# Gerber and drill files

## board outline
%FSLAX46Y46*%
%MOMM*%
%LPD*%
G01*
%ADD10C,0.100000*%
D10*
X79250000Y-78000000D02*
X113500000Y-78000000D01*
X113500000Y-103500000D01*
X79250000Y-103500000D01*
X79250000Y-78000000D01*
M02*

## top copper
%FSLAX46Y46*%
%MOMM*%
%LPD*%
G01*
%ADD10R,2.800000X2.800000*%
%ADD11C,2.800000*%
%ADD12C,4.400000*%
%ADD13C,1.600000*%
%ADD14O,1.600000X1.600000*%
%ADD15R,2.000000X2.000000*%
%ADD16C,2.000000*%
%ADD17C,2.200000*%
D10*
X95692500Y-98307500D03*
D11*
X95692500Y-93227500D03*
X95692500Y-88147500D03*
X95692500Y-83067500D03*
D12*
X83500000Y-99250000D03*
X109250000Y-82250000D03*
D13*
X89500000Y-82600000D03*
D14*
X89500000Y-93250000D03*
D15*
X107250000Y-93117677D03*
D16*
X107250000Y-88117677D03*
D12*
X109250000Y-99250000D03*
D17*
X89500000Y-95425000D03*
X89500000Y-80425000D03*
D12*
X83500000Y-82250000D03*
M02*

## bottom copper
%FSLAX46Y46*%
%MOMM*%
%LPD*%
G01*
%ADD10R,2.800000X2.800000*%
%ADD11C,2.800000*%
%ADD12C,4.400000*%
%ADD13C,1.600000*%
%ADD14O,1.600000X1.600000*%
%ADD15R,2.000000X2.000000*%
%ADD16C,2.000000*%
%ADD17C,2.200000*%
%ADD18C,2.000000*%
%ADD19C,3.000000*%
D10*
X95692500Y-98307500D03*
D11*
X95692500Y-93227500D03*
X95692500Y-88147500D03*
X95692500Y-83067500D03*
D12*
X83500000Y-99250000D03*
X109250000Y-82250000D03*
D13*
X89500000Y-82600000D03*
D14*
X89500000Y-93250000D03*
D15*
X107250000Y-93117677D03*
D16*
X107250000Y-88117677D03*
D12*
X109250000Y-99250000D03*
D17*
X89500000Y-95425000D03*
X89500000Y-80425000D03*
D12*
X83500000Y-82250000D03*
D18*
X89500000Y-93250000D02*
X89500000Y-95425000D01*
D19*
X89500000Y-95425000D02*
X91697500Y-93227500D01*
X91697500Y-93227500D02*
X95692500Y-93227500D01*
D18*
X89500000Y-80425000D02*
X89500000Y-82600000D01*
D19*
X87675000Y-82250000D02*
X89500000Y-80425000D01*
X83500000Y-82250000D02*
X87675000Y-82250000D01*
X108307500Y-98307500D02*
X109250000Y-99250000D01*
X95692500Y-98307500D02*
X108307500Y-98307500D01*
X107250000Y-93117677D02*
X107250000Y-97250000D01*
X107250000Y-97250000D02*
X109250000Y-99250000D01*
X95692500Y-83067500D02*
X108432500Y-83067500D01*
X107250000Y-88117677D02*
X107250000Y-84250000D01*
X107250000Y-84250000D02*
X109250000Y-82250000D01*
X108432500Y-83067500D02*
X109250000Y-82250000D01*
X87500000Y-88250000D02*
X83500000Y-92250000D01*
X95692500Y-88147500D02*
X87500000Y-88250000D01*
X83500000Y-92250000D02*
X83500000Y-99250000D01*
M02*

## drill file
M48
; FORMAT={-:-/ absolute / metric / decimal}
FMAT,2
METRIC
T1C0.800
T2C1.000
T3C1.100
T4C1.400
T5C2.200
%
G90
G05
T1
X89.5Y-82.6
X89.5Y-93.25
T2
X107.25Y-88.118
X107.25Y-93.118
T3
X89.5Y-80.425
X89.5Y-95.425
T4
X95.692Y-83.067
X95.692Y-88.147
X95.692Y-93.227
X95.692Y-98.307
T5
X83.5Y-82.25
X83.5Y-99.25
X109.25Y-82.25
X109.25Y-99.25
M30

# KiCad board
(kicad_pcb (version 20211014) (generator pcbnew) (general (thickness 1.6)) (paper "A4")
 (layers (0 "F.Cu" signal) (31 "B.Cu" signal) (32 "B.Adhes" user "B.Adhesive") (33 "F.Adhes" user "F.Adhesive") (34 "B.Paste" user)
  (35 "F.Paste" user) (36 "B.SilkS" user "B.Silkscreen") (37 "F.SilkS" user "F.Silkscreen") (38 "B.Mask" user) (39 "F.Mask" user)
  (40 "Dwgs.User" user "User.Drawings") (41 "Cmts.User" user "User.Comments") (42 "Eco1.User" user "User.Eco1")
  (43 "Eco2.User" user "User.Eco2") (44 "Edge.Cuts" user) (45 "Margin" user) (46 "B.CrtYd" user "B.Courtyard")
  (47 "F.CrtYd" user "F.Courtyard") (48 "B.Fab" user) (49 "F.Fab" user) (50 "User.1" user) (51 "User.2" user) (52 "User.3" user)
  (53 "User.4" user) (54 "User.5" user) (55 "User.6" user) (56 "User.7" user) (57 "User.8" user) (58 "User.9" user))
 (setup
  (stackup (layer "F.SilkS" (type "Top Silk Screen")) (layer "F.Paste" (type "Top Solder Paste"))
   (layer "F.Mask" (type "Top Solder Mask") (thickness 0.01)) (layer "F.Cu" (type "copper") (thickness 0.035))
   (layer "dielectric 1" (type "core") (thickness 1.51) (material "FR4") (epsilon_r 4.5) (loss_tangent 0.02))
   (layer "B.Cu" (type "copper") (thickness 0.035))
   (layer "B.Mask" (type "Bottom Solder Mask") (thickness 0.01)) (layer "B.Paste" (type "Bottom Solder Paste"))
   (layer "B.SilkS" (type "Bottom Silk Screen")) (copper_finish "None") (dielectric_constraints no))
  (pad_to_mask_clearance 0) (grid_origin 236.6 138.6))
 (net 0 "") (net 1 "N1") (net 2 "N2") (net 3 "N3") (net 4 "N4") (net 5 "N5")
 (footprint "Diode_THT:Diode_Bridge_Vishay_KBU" (layer "F.Cu") (at 95.6925 98.3075 90)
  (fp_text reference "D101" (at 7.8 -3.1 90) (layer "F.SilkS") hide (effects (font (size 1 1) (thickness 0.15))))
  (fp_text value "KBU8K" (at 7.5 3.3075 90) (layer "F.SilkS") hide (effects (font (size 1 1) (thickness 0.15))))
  (pad "1" thru_hole rect (at 0 0 90) (size 2.8 2.8) (drill 1.4) (layers *.Cu *.Mask) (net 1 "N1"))
  (pad "2" thru_hole circle (at 5.08 0 90) (size 2.8 2.8) (drill 1.4) (layers *.Cu *.Mask) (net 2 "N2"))
  (pad "3" thru_hole circle (at 10.16 0 90) (size 2.8 2.8) (drill 1.4) (layers *.Cu *.Mask) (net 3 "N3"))
  (pad "4" thru_hole circle (at 15.24 0 90) (size 2.8 2.8) (drill 1.4) (layers *.Cu *.Mask) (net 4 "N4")))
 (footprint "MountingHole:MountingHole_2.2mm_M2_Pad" (layer "F.Cu") (at 83.5 99.25)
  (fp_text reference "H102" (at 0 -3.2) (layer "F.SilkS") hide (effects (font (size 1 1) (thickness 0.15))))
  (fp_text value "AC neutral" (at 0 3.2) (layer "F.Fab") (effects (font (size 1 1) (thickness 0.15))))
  (pad "1" thru_hole circle (at 0 0) (size 4.4 4.4) (drill 2.2) (layers *.Cu *.Mask) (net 3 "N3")))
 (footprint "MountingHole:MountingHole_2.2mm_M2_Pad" (layer "F.Cu") (at 109.25 82.25 180)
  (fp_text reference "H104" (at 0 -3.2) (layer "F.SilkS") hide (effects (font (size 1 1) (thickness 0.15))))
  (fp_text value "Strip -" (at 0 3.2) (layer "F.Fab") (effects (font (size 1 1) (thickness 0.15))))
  (pad "1" thru_hole circle (at 0 0 180) (size 4.4 4.4) (drill 2.2) (layers *.Cu *.Mask) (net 4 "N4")))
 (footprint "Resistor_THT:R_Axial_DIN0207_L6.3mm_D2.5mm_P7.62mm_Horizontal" (layer "F.Cu") (at 89.5 84.1 -90)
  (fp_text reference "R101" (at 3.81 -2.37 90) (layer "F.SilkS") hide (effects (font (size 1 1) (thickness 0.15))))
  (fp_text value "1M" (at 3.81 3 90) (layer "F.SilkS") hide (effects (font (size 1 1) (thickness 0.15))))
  (pad "1" thru_hole circle (at -1.5 0 270) (size 1.6 1.6) (drill 0.8) (layers *.Cu *.Mask) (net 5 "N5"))
  (pad "2" thru_hole oval (at 9.15 0 270) (size 1.6 1.6) (drill 0.8) (layers *.Cu *.Mask) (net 2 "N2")))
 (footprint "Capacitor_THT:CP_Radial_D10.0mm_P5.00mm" (layer "F.Cu") (at 107.25 93.117677 90)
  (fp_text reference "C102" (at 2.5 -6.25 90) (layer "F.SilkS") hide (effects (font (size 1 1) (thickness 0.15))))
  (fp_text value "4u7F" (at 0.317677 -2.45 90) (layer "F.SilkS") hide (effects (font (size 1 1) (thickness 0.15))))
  (pad "1" thru_hole rect (at 0 0 90) (size 2 2) (drill 1) (layers *.Cu *.Mask) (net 1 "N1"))
  (pad "2" thru_hole circle (at 5 0 90) (size 2 2) (drill 1) (layers *.Cu *.Mask) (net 4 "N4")))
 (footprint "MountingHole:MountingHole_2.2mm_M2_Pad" (layer "F.Cu") (at 109.25 99.25)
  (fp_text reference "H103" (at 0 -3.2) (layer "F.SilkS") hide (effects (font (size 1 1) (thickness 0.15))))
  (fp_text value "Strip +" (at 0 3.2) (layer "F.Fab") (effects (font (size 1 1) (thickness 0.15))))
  (pad "1" thru_hole circle (at 0 0) (size 4.4 4.4) (drill 2.2) (layers *.Cu *.Mask) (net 1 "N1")))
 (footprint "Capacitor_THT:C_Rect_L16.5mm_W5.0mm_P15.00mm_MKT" (layer "F.Cu") (at 89.5 95.425 90)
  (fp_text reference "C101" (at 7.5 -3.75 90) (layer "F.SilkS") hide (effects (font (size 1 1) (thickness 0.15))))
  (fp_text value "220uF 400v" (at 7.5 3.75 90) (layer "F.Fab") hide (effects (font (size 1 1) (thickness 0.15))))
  (pad "1" thru_hole circle (at 0 0 90) (size 2.2 2.2) (drill 1.1) (layers *.Cu *.Mask) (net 2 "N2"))
  (pad "2" thru_hole circle (at 15 0 90) (size 2.2 2.2) (drill 1.1) (layers *.Cu *.Mask) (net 5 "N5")))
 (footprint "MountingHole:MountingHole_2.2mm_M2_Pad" (layer "F.Cu") (at 83.5 82.25)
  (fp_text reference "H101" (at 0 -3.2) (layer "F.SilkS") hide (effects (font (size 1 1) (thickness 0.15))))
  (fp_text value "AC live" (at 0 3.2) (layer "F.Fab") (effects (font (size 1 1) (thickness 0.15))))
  (pad "1" thru_hole circle (at 0 0) (size 4.4 4.4) (drill 2.2) (layers *.Cu *.Mask) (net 5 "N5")))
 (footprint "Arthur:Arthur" (layer "B.Cu") (at 101.4 90.6 180)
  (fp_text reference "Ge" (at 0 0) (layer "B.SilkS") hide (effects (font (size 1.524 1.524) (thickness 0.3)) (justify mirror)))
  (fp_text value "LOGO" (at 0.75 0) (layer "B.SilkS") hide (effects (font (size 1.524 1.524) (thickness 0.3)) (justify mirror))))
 (gr_rect (start 79.25 78) (end 113.5 103.5) (layer "Edge.Cuts") (width 0.1) (fill none))
 (segment (start 89.5 93.25) (end 89.5 95.425) (width 2) (layer "B.Cu") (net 2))
 (segment (start 89.5 95.425) (end 91.6975 93.2275) (width 3) (layer "B.Cu") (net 2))
 (segment (start 91.6975 93.2275) (end 95.6925 93.2275) (width 3) (layer "B.Cu") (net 2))
 (segment (start 89.5 80.425) (end 89.5 82.6) (width 2) (layer "B.Cu") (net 5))
 (segment (start 87.675 82.25) (end 89.5 80.425) (width 3) (layer "B.Cu") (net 5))
 (segment (start 83.5 82.25) (end 87.675 82.25) (width 3) (layer "B.Cu") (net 5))
 (segment (start 108.3075 98.3075) (end 109.25 99.25) (width 3) (layer "B.Cu") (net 1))
 (segment (start 95.6925 98.3075) (end 108.3075 98.3075) (width 3) (layer "B.Cu") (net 1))
 (segment (start 107.25 93.117677) (end 107.25 97.25) (width 3) (layer "B.Cu") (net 1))
 (segment (start 107.25 97.25) (end 109.25 99.25) (width 3) (layer "B.Cu") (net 1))
 (segment (start 95.6925 83.0675) (end 108.4325 83.0675) (width 3) (layer "B.Cu") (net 4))
 (segment (start 107.25 88.117677) (end 107.25 84.25) (width 3) (layer "B.Cu") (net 4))
 (segment (start 107.25 84.25) (end 109.25 82.25) (width 3) (layer "B.Cu") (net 4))
 (segment (start 108.4325 83.0675) (end 109.25 82.25) (width 3) (layer "B.Cu") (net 4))
 (segment (start 87.5 88.25) (end 83.5 92.25) (width 3) (layer "B.Cu") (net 3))
 (segment (start 95.6925 88.1475) (end 87.5 88.25) (width 3) (layer "B.Cu") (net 3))
 (segment (start 83.5 92.25) (end 83.5 99.25) (width 3) (layer "B.Cu") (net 3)))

